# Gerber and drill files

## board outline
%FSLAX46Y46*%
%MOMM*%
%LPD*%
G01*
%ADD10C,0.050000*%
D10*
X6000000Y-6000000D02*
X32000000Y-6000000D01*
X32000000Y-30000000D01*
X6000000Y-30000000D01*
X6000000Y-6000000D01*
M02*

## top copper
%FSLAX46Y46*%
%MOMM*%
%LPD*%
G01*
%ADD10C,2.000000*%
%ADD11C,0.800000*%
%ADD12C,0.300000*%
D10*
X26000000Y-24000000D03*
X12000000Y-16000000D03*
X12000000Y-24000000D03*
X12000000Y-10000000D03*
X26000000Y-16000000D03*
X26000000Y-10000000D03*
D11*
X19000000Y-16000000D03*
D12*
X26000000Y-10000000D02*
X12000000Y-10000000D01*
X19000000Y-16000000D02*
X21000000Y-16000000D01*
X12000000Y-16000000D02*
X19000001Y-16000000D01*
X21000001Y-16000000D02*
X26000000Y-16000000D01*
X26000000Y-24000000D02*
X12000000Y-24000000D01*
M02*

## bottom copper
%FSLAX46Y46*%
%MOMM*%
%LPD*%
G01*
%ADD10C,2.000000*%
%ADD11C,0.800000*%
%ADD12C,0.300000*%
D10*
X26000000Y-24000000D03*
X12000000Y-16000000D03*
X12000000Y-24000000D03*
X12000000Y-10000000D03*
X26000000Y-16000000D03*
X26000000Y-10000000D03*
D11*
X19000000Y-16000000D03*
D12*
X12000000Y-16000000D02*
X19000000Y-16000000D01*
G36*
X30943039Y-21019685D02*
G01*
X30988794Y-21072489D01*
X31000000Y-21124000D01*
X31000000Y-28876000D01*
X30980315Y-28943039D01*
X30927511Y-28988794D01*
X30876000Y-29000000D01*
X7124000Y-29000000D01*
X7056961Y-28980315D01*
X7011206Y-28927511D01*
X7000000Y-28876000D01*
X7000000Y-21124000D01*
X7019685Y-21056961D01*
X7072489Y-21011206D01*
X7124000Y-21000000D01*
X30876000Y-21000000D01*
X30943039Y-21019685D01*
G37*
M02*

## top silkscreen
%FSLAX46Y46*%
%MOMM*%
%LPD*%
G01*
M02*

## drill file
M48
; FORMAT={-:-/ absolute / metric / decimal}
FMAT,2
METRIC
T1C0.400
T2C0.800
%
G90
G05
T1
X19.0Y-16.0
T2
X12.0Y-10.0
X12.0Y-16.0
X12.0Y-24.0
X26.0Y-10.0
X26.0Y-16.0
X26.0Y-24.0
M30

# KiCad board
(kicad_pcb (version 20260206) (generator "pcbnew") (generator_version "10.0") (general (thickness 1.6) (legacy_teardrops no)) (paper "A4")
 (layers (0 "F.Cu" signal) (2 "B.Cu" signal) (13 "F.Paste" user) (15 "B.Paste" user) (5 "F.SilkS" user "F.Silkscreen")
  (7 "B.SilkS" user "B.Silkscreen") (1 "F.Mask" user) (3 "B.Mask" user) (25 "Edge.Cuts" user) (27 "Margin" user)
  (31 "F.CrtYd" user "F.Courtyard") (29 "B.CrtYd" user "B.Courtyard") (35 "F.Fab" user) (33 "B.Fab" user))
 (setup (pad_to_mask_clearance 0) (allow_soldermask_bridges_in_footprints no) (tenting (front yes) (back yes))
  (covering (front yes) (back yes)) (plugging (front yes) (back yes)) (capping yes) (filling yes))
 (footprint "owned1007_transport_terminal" (layer "F.Cu") (at 26 24)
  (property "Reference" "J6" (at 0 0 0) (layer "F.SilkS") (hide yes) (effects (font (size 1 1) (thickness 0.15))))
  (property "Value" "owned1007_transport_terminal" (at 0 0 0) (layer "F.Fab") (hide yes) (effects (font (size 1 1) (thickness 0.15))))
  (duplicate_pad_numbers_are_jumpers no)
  (pad "1" thru_hole circle (at 0 0) (size 2 2) (drill 0.8) (layers "*.Cu" "*.Mask") (remove_unused_layers no) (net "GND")))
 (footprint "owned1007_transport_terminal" (layer "F.Cu") (at 12 16)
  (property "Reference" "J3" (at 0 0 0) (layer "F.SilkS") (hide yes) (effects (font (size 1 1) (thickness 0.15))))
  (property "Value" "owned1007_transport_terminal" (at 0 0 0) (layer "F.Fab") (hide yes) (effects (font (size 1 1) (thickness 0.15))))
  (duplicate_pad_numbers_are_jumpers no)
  (pad "1" thru_hole circle (at 0 0) (size 2 2) (drill 0.8) (layers "*.Cu" "*.Mask") (remove_unused_layers no) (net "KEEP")))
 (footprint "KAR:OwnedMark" (layer "F.Cu") (at 10 28)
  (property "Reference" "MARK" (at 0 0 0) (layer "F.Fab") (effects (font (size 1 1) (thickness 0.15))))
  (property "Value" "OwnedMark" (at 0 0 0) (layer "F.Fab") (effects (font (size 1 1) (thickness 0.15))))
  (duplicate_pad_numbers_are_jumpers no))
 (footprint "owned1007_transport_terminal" (layer "F.Cu") (at 12 24)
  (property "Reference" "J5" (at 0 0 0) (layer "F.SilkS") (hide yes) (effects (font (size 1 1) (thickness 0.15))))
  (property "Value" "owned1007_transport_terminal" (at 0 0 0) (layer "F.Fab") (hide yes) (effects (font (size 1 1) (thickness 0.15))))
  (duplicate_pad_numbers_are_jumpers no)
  (pad "1" thru_hole circle (at 0 0) (size 2 2) (drill 0.8) (layers "*.Cu" "*.Mask") (remove_unused_layers no) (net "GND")))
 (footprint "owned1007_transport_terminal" (layer "F.Cu") (at 12 10)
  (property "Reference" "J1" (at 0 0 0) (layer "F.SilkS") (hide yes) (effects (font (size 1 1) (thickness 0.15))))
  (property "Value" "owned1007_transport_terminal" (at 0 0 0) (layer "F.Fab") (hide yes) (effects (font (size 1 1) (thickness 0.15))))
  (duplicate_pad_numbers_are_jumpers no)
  (pad "1" thru_hole circle (at 0 0) (size 2 2) (drill 0.8) (layers "*.Cu" "*.Mask") (remove_unused_layers no) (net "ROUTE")))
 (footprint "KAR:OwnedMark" (layer "F.Cu") (at 13 28)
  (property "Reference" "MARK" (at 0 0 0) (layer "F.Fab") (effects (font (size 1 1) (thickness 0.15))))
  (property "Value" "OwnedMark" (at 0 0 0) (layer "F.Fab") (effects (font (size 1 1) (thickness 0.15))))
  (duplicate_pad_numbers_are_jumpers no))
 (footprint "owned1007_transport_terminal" (layer "F.Cu") (at 26 16)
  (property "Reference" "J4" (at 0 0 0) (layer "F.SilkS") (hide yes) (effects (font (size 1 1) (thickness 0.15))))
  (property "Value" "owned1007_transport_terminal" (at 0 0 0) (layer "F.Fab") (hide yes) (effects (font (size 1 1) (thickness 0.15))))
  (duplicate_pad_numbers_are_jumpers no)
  (pad "1" thru_hole circle (at 0 0) (size 2 2) (drill 0.8) (layers "*.Cu" "*.Mask") (remove_unused_layers no) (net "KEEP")))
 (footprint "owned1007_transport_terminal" (layer "F.Cu") (at 26 10)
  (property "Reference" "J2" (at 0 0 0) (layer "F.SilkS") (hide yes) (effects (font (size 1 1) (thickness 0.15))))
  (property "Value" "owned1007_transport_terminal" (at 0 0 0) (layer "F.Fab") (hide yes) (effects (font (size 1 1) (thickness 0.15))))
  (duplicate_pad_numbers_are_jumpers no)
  (pad "1" thru_hole circle (at 0 0) (size 2 2) (drill 0.8) (layers "*.Cu" "*.Mask") (remove_unused_layers no) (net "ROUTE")))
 (gr_rect (start 6 6) (end 32 30) (stroke (width 0.05) (type default)) (fill no) (layer "Edge.Cuts"))
 (segment (start 26 10) (end 12 10) (width 0.3) (layer "F.Cu") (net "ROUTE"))
 (segment (start 19 16) (end 21 16) (width 0.3) (layer "F.Cu") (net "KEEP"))
 (segment (start 12 16) (end 19.000001 16) (width 0.3) (layer "F.Cu") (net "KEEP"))
 (segment (start 21.000001 16) (end 26 16) (width 0.3) (layer "F.Cu") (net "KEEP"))
 (via (at 19 16) (size 0.8) (drill 0.4) (layers "F.Cu" "B.Cu") (free yes) (capping no) (covering (front no) (back no))
  (plugging (front no) (back no)) (filling no) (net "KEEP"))
 (segment (start 12 16) (end 19 16) (width 0.3) (locked yes) (layer "B.Cu") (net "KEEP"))
 (segment (start 26 24) (end 12 24) (width 0.3) (layer "F.Cu") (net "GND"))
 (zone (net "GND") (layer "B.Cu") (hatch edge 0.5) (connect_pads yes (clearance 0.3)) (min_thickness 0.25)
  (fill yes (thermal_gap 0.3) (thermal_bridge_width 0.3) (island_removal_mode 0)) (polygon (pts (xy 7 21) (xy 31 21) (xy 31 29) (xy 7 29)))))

